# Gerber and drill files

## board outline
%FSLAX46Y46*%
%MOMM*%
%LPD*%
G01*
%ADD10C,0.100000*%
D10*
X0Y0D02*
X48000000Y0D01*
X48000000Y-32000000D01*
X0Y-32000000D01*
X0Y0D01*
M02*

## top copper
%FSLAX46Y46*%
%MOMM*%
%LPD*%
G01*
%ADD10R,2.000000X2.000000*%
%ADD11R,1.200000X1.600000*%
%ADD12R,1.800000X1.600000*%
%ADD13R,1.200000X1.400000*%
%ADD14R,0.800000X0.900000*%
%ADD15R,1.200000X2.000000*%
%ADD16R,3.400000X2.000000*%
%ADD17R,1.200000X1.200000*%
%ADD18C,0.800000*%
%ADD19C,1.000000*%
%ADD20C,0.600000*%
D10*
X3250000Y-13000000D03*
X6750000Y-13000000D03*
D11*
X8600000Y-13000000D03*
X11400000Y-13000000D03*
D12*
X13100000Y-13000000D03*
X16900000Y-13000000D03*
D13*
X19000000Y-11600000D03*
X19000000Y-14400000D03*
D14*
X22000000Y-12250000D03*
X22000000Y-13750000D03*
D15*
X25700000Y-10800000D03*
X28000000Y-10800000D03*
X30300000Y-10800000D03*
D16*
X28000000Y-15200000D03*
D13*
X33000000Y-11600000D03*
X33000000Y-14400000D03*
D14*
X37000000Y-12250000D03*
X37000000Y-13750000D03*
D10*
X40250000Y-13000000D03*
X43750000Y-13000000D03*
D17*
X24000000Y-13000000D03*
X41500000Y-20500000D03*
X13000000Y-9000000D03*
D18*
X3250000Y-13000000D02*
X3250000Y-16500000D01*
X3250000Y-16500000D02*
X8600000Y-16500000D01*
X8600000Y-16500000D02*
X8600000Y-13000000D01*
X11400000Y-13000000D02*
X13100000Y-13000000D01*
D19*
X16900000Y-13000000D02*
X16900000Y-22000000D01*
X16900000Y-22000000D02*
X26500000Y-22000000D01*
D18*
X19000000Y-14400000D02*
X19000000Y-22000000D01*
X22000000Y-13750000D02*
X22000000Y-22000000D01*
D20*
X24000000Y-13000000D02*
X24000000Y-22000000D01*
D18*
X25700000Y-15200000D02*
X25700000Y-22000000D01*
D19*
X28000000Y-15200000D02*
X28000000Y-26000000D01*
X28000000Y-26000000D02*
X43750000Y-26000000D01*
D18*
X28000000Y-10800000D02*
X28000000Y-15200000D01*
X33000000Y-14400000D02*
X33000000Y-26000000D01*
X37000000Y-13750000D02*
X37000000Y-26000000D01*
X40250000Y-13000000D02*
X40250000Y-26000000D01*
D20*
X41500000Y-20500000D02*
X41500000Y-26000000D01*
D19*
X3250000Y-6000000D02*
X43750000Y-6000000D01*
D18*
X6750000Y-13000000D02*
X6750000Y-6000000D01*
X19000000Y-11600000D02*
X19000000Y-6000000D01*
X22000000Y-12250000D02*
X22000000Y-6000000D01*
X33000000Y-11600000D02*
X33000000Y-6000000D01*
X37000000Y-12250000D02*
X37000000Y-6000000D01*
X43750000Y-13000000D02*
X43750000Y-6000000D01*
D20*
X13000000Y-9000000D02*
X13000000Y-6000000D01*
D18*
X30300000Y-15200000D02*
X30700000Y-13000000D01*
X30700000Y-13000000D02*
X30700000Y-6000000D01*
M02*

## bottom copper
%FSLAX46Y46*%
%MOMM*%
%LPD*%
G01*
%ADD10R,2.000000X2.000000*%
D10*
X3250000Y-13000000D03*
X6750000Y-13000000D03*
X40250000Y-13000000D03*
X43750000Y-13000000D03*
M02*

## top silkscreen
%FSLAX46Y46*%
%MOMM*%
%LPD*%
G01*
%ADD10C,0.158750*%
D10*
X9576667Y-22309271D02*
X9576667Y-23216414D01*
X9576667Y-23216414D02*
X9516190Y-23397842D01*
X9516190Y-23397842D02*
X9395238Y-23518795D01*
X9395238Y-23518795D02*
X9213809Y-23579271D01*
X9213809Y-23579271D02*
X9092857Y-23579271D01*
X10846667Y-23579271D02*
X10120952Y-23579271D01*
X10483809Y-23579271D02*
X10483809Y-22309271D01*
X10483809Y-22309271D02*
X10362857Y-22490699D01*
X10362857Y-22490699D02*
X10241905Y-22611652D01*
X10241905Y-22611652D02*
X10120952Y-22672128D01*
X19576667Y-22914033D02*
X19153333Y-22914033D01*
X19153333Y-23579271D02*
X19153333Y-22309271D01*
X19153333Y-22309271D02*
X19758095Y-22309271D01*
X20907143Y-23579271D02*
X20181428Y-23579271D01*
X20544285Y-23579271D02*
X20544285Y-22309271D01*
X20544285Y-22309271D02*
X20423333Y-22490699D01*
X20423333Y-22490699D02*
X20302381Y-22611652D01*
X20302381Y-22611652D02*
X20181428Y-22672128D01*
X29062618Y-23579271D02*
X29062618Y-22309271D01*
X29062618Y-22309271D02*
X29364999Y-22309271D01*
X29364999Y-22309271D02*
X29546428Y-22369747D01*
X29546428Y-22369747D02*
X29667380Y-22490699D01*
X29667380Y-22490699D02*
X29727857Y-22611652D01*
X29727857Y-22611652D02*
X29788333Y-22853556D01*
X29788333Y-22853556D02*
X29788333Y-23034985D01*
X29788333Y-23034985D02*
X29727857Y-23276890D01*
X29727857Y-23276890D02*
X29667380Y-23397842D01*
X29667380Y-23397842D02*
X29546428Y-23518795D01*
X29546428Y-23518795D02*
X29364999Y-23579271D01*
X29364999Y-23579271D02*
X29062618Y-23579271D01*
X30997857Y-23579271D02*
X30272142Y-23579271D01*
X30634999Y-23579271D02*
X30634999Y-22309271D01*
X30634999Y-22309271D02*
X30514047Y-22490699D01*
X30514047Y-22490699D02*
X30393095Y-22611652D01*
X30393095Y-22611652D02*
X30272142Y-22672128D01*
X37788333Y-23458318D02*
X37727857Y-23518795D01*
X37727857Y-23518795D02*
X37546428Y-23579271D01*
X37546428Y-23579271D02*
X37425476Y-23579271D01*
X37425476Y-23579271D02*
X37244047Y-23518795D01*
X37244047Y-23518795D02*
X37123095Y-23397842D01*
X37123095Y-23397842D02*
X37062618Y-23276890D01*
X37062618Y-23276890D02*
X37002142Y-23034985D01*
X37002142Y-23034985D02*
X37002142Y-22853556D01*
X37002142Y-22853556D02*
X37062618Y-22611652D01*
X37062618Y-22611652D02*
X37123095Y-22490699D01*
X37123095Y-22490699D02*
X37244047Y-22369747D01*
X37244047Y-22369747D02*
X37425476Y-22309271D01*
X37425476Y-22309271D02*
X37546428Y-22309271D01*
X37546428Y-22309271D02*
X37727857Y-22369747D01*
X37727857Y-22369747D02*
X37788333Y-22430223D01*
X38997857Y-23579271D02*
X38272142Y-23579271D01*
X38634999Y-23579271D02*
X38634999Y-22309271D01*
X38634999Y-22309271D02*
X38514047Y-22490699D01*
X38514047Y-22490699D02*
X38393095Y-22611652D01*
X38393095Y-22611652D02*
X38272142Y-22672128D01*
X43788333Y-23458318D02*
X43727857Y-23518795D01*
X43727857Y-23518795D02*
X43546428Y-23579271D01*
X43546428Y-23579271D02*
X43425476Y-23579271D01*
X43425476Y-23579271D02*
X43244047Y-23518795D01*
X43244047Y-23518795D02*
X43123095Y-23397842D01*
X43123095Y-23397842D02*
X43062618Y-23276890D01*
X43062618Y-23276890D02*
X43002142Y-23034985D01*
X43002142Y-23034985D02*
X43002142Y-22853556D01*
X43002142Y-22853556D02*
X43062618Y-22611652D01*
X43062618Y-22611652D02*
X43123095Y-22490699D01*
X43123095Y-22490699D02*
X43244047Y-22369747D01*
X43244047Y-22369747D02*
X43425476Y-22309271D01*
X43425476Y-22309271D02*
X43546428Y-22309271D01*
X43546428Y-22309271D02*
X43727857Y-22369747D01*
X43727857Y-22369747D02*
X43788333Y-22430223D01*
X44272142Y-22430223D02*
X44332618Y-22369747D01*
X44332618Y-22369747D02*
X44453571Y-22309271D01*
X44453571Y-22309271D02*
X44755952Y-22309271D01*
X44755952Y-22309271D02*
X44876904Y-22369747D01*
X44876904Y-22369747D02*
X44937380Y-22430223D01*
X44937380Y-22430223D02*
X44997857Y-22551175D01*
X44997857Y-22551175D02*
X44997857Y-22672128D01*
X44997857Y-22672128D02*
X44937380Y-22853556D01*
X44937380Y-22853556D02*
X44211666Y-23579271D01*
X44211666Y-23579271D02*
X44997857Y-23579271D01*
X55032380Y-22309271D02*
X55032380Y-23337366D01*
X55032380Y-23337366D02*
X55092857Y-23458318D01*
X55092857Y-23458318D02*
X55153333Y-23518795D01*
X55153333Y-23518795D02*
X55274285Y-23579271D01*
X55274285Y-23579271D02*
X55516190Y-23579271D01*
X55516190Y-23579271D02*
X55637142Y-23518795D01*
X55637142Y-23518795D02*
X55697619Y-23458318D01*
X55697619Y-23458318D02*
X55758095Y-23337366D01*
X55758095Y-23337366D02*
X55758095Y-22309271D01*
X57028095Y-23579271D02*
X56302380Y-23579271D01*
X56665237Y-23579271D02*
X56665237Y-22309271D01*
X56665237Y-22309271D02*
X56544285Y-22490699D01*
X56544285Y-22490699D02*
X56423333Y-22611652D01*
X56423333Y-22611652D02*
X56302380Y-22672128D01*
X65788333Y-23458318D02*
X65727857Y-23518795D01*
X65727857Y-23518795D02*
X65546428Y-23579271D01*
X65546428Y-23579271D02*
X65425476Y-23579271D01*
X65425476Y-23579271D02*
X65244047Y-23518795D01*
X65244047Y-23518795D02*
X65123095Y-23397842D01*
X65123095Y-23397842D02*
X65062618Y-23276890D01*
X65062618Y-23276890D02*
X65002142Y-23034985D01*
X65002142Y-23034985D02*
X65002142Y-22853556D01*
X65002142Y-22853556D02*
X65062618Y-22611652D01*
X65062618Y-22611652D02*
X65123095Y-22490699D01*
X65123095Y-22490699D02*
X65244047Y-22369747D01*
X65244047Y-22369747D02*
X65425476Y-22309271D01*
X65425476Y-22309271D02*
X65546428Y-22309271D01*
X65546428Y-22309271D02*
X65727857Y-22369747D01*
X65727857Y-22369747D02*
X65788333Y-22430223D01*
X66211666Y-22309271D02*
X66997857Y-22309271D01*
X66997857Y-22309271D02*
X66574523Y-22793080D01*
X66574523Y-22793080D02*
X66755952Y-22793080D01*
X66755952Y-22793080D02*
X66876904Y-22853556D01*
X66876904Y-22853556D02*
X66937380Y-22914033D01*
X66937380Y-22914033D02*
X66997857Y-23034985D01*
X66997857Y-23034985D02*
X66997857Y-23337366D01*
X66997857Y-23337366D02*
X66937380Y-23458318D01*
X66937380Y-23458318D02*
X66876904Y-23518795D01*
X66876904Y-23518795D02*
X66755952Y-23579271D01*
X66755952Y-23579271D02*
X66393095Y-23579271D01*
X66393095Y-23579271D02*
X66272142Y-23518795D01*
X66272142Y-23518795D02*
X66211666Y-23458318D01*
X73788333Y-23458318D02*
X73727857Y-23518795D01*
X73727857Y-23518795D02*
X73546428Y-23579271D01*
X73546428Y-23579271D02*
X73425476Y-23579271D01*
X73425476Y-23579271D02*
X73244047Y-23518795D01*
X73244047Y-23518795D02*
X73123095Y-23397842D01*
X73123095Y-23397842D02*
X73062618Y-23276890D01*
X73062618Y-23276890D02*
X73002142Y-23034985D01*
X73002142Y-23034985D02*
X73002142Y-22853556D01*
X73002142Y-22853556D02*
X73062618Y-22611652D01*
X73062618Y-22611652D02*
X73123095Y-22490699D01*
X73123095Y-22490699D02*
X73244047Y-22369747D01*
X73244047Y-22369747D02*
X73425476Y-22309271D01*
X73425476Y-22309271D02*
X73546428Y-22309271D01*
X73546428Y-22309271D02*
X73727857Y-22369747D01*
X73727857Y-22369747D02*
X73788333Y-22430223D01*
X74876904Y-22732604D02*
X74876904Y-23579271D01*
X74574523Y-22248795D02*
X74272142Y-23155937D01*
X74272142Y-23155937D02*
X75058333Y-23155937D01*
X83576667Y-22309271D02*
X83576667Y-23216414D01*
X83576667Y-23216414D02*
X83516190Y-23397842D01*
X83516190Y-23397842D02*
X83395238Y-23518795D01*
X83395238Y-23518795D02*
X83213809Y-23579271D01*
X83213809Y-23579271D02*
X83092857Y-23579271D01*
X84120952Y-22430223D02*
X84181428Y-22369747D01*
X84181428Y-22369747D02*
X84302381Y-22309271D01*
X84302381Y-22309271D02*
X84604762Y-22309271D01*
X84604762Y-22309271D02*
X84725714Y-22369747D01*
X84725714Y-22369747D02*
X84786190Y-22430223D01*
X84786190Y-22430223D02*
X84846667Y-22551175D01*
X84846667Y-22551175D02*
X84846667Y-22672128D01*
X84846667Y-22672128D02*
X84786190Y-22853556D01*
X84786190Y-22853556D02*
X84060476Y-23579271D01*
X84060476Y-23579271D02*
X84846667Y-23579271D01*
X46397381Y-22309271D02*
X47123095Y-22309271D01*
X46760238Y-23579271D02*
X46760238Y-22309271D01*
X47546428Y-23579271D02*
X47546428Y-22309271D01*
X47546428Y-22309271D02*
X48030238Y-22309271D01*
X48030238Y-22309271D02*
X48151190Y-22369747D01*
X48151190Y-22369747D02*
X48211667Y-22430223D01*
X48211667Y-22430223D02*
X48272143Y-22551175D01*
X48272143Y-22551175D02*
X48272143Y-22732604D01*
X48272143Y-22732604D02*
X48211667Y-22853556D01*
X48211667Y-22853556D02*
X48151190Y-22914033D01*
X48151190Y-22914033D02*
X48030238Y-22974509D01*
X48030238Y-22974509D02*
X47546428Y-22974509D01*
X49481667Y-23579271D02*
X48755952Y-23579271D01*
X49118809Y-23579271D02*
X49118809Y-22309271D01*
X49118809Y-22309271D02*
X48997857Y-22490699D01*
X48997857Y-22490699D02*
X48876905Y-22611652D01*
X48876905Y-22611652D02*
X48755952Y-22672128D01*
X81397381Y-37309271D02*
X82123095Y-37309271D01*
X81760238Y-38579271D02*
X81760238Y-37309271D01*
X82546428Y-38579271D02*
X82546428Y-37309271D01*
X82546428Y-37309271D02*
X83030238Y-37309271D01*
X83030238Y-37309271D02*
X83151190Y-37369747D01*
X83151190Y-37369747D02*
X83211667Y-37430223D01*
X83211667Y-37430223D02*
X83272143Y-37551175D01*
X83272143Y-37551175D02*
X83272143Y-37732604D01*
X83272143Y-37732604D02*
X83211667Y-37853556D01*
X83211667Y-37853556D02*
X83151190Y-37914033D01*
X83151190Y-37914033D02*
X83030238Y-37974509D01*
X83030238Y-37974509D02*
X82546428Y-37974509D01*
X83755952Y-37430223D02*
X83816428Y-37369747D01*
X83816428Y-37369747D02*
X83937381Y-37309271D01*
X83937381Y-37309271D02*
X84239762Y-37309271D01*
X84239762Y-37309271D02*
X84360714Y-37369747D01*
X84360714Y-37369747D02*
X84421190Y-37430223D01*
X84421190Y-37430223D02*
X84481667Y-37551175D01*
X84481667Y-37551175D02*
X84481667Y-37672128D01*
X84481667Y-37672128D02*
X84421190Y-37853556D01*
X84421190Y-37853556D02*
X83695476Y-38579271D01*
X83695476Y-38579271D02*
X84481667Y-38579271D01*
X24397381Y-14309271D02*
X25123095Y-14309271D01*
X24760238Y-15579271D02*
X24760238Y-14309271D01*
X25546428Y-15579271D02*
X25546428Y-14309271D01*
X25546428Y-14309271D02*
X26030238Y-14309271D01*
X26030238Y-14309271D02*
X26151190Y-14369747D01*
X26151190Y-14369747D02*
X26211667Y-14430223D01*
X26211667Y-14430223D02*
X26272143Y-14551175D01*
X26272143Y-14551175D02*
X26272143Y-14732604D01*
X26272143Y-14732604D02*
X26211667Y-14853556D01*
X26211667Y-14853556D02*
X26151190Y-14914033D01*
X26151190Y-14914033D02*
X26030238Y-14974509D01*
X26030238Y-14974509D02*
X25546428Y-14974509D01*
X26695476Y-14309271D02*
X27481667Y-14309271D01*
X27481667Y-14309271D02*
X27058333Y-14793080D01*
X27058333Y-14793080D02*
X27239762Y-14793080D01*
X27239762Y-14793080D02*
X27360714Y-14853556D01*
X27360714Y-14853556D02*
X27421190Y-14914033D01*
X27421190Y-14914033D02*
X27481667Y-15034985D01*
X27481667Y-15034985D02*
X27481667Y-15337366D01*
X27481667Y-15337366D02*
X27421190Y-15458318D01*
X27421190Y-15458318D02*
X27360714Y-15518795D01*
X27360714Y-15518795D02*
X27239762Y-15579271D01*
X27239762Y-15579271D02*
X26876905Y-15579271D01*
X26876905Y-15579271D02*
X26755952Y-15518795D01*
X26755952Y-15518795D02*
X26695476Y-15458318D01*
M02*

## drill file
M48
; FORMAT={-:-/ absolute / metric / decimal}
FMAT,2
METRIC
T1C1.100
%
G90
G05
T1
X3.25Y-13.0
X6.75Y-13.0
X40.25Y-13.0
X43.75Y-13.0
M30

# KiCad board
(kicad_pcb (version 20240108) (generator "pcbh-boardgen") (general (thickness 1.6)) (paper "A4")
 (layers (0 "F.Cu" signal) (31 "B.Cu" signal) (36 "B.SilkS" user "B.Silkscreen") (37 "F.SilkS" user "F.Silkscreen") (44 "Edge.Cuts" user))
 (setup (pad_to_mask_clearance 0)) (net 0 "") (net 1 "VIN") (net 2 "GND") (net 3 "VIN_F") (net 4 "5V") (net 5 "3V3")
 (gr_rect (start 0 0) (end 48.0 32.0) (stroke (width 0.1) (type default)) (fill none) (layer "Edge.Cuts"))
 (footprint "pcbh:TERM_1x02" (layer "F.Cu") (at 5.0 13.0 0)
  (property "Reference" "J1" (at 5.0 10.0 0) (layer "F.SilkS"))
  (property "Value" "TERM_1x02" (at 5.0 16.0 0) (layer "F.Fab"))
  (pad "1" thru_hole rect (at -1.75 0 0) (size 2.0 2.0) (drill 1.1) (layers "*.Cu" "*.Mask") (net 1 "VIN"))
  (pad "2" thru_hole rect (at 1.75 0 0) (size 2.0 2.0) (drill 1.1) (layers "*.Cu" "*.Mask") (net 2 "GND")))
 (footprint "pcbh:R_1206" (layer "F.Cu") (at 10.0 13.0 0)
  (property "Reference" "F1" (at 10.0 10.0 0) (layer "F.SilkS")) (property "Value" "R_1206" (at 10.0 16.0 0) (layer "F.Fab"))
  (pad "1" smd rect (at -1.4 0 0) (size 1.2 1.6) (layers "F.Cu" "F.Paste" "F.Mask") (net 1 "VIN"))
  (pad "2" smd rect (at 1.4 0 0) (size 1.2 1.6) (layers "F.Cu" "F.Paste" "F.Mask") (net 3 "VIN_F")))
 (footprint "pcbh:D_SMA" (layer "F.Cu") (at 15.0 13.0 0)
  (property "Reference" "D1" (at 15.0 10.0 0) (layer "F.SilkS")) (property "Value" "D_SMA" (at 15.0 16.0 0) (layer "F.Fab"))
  (pad "1" smd rect (at -1.9 0 0) (size 1.8 1.6) (layers "F.Cu" "F.Paste" "F.Mask") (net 3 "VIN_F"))
  (pad "2" smd rect (at 1.9 0 0) (size 1.8 1.6) (layers "F.Cu" "F.Paste" "F.Mask") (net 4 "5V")))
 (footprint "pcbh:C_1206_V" (layer "F.Cu") (at 19.0 13.0 0)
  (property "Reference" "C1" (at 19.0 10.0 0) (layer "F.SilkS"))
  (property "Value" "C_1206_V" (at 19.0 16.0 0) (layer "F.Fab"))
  (pad "1" smd rect (at 0 -1.4 0) (size 1.2 1.4) (layers "F.Cu" "F.Paste" "F.Mask") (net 2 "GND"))
  (pad "2" smd rect (at 0 1.4 0) (size 1.2 1.4) (layers "F.Cu" "F.Paste" "F.Mask") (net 4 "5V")))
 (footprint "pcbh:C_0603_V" (layer "F.Cu") (at 22.0 13.0 0)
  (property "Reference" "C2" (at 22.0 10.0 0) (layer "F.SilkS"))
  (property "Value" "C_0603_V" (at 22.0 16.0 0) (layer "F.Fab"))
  (pad "1" smd rect (at 0 -0.75 0) (size 0.8 0.9) (layers "F.Cu" "F.Paste" "F.Mask") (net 2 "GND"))
  (pad "2" smd rect (at 0 0.75 0) (size 0.8 0.9) (layers "F.Cu" "F.Paste" "F.Mask") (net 4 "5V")))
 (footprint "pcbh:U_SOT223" (layer "F.Cu") (at 28.0 13.0 0)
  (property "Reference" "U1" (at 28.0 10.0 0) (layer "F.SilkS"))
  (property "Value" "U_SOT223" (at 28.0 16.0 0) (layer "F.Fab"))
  (pad "1" smd rect (at -2.3 -2.2 0) (size 1.2 2.0) (layers "F.Cu" "F.Paste" "F.Mask") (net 2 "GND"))
  (pad "2" smd rect (at 0.0 -2.2 0) (size 1.2 2.0) (layers "F.Cu" "F.Paste" "F.Mask") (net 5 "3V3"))
  (pad "3" smd rect (at 2.3 -2.2 0) (size 1.2 2.0) (layers "F.Cu" "F.Paste" "F.Mask") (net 4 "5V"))
  (pad "4" smd rect (at 0.0 2.2 0) (size 3.4 2.0) (layers "F.Cu" "F.Paste" "F.Mask") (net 5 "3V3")))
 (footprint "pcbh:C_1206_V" (layer "F.Cu") (at 33.0 13.0 0)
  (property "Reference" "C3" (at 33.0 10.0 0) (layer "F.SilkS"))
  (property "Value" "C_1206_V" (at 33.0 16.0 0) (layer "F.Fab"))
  (pad "1" smd rect (at 0 -1.4 0) (size 1.2 1.4) (layers "F.Cu" "F.Paste" "F.Mask") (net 2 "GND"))
  (pad "2" smd rect (at 0 1.4 0) (size 1.2 1.4) (layers "F.Cu" "F.Paste" "F.Mask") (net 5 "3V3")))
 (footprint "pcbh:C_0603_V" (layer "F.Cu") (at 37.0 13.0 0)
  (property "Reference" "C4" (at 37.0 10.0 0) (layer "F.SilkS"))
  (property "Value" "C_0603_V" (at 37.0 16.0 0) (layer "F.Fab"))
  (pad "1" smd rect (at 0 -0.75 0) (size 0.8 0.9) (layers "F.Cu" "F.Paste" "F.Mask") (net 2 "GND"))
  (pad "2" smd rect (at 0 0.75 0) (size 0.8 0.9) (layers "F.Cu" "F.Paste" "F.Mask") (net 5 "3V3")))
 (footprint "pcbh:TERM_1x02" (layer "F.Cu") (at 42.0 13.0 0)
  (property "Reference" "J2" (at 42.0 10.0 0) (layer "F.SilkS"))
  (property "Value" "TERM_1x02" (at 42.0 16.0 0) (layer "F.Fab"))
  (pad "1" thru_hole rect (at -1.75 0 0) (size 2.0 2.0) (drill 1.1) (layers "*.Cu" "*.Mask") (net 5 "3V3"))
  (pad "2" thru_hole rect (at 1.75 0 0) (size 2.0 2.0) (drill 1.1) (layers "*.Cu" "*.Mask") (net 2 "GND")))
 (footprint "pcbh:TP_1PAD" (layer "F.Cu") (at 24.0 13.0 0)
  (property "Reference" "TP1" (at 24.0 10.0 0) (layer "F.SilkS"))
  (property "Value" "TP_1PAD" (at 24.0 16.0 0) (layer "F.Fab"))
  (pad "1" smd rect (at 0 0 0) (size 1.2 1.2) (layers "F.Cu" "F.Paste" "F.Mask") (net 4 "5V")))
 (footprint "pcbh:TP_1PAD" (layer "F.Cu") (at 41.5 20.5 0)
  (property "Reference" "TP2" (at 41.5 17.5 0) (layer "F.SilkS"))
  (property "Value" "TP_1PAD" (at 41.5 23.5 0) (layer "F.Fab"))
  (pad "1" smd rect (at 0 0 0) (size 1.2 1.2) (layers "F.Cu" "F.Paste" "F.Mask") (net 5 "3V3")))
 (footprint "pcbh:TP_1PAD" (layer "F.Cu") (at 13.0 9.0 0)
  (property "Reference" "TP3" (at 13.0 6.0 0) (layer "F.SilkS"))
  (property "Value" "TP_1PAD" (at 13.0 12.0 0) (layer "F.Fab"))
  (pad "1" smd rect (at 0 0 0) (size 1.2 1.2) (layers "F.Cu" "F.Paste" "F.Mask") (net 2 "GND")))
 (segment (start 3.25 13.0) (end 3.25 16.5) (width 0.8) (layer "F.Cu") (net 1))
 (segment (start 3.25 16.5) (end 8.6 16.5) (width 0.8) (layer "F.Cu") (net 1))
 (segment (start 8.6 16.5) (end 8.6 13.0) (width 0.8) (layer "F.Cu") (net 1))
 (segment (start 11.4 13.0) (end 13.1 13.0) (width 0.8) (layer "F.Cu") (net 3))
 (segment (start 16.9 13.0) (end 16.9 22.0) (width 1.0) (layer "F.Cu") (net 4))
 (segment (start 16.9 22.0) (end 26.5 22.0) (width 1.0) (layer "F.Cu") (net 4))
 (segment (start 19.0 14.4) (end 19.0 22.0) (width 0.8) (layer "F.Cu") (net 4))
 (segment (start 22.0 13.75) (end 22.0 22.0) (width 0.8) (layer "F.Cu") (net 4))
 (segment (start 24.0 13.0) (end 24.0 22.0) (width 0.6) (layer "F.Cu") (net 4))
 (segment (start 25.7 15.2) (end 25.7 22.0) (width 0.8) (layer "F.Cu") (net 4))
 (segment (start 28.0 15.2) (end 28.0 26.0) (width 1.0) (layer "F.Cu") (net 5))
 (segment (start 28.0 26.0) (end 43.75 26.0) (width 1.0) (layer "F.Cu") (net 5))
 (segment (start 28.0 10.8) (end 28.0 15.2) (width 0.8) (layer "F.Cu") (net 5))
 (segment (start 33.0 14.4) (end 33.0 26.0) (width 0.8) (layer "F.Cu") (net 5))
 (segment (start 37.0 13.75) (end 37.0 26.0) (width 0.8) (layer "F.Cu") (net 5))
 (segment (start 40.25 13.0) (end 40.25 26.0) (width 0.8) (layer "F.Cu") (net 5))
 (segment (start 41.5 20.5) (end 41.5 26.0) (width 0.6) (layer "F.Cu") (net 5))
 (segment (start 3.25 6.0) (end 43.75 6.0) (width 1.0) (layer "F.Cu") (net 2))
 (segment (start 6.75 13.0) (end 6.75 6.0) (width 0.8) (layer "F.Cu") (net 2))
 (segment (start 19.0 11.6) (end 19.0 6.0) (width 0.8) (layer "F.Cu") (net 2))
 (segment (start 22.0 12.25) (end 22.0 6.0) (width 0.8) (layer "F.Cu") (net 2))
 (segment (start 33.0 11.6) (end 33.0 6.0) (width 0.8) (layer "F.Cu") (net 2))
 (segment (start 37.0 12.25) (end 37.0 6.0) (width 0.8) (layer "F.Cu") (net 2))
 (segment (start 43.75 13.0) (end 43.75 6.0) (width 0.8) (layer "F.Cu") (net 2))
 (segment (start 13.0 9.0) (end 13.0 6.0) (width 0.6) (layer "F.Cu") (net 2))
 (segment (start 30.3 15.2) (end 30.7 13.0) (width 0.8) (layer "F.Cu") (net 2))
 (segment (start 30.7 13.0) (end 30.7 6.0) (width 0.8) (layer "F.Cu") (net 2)))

